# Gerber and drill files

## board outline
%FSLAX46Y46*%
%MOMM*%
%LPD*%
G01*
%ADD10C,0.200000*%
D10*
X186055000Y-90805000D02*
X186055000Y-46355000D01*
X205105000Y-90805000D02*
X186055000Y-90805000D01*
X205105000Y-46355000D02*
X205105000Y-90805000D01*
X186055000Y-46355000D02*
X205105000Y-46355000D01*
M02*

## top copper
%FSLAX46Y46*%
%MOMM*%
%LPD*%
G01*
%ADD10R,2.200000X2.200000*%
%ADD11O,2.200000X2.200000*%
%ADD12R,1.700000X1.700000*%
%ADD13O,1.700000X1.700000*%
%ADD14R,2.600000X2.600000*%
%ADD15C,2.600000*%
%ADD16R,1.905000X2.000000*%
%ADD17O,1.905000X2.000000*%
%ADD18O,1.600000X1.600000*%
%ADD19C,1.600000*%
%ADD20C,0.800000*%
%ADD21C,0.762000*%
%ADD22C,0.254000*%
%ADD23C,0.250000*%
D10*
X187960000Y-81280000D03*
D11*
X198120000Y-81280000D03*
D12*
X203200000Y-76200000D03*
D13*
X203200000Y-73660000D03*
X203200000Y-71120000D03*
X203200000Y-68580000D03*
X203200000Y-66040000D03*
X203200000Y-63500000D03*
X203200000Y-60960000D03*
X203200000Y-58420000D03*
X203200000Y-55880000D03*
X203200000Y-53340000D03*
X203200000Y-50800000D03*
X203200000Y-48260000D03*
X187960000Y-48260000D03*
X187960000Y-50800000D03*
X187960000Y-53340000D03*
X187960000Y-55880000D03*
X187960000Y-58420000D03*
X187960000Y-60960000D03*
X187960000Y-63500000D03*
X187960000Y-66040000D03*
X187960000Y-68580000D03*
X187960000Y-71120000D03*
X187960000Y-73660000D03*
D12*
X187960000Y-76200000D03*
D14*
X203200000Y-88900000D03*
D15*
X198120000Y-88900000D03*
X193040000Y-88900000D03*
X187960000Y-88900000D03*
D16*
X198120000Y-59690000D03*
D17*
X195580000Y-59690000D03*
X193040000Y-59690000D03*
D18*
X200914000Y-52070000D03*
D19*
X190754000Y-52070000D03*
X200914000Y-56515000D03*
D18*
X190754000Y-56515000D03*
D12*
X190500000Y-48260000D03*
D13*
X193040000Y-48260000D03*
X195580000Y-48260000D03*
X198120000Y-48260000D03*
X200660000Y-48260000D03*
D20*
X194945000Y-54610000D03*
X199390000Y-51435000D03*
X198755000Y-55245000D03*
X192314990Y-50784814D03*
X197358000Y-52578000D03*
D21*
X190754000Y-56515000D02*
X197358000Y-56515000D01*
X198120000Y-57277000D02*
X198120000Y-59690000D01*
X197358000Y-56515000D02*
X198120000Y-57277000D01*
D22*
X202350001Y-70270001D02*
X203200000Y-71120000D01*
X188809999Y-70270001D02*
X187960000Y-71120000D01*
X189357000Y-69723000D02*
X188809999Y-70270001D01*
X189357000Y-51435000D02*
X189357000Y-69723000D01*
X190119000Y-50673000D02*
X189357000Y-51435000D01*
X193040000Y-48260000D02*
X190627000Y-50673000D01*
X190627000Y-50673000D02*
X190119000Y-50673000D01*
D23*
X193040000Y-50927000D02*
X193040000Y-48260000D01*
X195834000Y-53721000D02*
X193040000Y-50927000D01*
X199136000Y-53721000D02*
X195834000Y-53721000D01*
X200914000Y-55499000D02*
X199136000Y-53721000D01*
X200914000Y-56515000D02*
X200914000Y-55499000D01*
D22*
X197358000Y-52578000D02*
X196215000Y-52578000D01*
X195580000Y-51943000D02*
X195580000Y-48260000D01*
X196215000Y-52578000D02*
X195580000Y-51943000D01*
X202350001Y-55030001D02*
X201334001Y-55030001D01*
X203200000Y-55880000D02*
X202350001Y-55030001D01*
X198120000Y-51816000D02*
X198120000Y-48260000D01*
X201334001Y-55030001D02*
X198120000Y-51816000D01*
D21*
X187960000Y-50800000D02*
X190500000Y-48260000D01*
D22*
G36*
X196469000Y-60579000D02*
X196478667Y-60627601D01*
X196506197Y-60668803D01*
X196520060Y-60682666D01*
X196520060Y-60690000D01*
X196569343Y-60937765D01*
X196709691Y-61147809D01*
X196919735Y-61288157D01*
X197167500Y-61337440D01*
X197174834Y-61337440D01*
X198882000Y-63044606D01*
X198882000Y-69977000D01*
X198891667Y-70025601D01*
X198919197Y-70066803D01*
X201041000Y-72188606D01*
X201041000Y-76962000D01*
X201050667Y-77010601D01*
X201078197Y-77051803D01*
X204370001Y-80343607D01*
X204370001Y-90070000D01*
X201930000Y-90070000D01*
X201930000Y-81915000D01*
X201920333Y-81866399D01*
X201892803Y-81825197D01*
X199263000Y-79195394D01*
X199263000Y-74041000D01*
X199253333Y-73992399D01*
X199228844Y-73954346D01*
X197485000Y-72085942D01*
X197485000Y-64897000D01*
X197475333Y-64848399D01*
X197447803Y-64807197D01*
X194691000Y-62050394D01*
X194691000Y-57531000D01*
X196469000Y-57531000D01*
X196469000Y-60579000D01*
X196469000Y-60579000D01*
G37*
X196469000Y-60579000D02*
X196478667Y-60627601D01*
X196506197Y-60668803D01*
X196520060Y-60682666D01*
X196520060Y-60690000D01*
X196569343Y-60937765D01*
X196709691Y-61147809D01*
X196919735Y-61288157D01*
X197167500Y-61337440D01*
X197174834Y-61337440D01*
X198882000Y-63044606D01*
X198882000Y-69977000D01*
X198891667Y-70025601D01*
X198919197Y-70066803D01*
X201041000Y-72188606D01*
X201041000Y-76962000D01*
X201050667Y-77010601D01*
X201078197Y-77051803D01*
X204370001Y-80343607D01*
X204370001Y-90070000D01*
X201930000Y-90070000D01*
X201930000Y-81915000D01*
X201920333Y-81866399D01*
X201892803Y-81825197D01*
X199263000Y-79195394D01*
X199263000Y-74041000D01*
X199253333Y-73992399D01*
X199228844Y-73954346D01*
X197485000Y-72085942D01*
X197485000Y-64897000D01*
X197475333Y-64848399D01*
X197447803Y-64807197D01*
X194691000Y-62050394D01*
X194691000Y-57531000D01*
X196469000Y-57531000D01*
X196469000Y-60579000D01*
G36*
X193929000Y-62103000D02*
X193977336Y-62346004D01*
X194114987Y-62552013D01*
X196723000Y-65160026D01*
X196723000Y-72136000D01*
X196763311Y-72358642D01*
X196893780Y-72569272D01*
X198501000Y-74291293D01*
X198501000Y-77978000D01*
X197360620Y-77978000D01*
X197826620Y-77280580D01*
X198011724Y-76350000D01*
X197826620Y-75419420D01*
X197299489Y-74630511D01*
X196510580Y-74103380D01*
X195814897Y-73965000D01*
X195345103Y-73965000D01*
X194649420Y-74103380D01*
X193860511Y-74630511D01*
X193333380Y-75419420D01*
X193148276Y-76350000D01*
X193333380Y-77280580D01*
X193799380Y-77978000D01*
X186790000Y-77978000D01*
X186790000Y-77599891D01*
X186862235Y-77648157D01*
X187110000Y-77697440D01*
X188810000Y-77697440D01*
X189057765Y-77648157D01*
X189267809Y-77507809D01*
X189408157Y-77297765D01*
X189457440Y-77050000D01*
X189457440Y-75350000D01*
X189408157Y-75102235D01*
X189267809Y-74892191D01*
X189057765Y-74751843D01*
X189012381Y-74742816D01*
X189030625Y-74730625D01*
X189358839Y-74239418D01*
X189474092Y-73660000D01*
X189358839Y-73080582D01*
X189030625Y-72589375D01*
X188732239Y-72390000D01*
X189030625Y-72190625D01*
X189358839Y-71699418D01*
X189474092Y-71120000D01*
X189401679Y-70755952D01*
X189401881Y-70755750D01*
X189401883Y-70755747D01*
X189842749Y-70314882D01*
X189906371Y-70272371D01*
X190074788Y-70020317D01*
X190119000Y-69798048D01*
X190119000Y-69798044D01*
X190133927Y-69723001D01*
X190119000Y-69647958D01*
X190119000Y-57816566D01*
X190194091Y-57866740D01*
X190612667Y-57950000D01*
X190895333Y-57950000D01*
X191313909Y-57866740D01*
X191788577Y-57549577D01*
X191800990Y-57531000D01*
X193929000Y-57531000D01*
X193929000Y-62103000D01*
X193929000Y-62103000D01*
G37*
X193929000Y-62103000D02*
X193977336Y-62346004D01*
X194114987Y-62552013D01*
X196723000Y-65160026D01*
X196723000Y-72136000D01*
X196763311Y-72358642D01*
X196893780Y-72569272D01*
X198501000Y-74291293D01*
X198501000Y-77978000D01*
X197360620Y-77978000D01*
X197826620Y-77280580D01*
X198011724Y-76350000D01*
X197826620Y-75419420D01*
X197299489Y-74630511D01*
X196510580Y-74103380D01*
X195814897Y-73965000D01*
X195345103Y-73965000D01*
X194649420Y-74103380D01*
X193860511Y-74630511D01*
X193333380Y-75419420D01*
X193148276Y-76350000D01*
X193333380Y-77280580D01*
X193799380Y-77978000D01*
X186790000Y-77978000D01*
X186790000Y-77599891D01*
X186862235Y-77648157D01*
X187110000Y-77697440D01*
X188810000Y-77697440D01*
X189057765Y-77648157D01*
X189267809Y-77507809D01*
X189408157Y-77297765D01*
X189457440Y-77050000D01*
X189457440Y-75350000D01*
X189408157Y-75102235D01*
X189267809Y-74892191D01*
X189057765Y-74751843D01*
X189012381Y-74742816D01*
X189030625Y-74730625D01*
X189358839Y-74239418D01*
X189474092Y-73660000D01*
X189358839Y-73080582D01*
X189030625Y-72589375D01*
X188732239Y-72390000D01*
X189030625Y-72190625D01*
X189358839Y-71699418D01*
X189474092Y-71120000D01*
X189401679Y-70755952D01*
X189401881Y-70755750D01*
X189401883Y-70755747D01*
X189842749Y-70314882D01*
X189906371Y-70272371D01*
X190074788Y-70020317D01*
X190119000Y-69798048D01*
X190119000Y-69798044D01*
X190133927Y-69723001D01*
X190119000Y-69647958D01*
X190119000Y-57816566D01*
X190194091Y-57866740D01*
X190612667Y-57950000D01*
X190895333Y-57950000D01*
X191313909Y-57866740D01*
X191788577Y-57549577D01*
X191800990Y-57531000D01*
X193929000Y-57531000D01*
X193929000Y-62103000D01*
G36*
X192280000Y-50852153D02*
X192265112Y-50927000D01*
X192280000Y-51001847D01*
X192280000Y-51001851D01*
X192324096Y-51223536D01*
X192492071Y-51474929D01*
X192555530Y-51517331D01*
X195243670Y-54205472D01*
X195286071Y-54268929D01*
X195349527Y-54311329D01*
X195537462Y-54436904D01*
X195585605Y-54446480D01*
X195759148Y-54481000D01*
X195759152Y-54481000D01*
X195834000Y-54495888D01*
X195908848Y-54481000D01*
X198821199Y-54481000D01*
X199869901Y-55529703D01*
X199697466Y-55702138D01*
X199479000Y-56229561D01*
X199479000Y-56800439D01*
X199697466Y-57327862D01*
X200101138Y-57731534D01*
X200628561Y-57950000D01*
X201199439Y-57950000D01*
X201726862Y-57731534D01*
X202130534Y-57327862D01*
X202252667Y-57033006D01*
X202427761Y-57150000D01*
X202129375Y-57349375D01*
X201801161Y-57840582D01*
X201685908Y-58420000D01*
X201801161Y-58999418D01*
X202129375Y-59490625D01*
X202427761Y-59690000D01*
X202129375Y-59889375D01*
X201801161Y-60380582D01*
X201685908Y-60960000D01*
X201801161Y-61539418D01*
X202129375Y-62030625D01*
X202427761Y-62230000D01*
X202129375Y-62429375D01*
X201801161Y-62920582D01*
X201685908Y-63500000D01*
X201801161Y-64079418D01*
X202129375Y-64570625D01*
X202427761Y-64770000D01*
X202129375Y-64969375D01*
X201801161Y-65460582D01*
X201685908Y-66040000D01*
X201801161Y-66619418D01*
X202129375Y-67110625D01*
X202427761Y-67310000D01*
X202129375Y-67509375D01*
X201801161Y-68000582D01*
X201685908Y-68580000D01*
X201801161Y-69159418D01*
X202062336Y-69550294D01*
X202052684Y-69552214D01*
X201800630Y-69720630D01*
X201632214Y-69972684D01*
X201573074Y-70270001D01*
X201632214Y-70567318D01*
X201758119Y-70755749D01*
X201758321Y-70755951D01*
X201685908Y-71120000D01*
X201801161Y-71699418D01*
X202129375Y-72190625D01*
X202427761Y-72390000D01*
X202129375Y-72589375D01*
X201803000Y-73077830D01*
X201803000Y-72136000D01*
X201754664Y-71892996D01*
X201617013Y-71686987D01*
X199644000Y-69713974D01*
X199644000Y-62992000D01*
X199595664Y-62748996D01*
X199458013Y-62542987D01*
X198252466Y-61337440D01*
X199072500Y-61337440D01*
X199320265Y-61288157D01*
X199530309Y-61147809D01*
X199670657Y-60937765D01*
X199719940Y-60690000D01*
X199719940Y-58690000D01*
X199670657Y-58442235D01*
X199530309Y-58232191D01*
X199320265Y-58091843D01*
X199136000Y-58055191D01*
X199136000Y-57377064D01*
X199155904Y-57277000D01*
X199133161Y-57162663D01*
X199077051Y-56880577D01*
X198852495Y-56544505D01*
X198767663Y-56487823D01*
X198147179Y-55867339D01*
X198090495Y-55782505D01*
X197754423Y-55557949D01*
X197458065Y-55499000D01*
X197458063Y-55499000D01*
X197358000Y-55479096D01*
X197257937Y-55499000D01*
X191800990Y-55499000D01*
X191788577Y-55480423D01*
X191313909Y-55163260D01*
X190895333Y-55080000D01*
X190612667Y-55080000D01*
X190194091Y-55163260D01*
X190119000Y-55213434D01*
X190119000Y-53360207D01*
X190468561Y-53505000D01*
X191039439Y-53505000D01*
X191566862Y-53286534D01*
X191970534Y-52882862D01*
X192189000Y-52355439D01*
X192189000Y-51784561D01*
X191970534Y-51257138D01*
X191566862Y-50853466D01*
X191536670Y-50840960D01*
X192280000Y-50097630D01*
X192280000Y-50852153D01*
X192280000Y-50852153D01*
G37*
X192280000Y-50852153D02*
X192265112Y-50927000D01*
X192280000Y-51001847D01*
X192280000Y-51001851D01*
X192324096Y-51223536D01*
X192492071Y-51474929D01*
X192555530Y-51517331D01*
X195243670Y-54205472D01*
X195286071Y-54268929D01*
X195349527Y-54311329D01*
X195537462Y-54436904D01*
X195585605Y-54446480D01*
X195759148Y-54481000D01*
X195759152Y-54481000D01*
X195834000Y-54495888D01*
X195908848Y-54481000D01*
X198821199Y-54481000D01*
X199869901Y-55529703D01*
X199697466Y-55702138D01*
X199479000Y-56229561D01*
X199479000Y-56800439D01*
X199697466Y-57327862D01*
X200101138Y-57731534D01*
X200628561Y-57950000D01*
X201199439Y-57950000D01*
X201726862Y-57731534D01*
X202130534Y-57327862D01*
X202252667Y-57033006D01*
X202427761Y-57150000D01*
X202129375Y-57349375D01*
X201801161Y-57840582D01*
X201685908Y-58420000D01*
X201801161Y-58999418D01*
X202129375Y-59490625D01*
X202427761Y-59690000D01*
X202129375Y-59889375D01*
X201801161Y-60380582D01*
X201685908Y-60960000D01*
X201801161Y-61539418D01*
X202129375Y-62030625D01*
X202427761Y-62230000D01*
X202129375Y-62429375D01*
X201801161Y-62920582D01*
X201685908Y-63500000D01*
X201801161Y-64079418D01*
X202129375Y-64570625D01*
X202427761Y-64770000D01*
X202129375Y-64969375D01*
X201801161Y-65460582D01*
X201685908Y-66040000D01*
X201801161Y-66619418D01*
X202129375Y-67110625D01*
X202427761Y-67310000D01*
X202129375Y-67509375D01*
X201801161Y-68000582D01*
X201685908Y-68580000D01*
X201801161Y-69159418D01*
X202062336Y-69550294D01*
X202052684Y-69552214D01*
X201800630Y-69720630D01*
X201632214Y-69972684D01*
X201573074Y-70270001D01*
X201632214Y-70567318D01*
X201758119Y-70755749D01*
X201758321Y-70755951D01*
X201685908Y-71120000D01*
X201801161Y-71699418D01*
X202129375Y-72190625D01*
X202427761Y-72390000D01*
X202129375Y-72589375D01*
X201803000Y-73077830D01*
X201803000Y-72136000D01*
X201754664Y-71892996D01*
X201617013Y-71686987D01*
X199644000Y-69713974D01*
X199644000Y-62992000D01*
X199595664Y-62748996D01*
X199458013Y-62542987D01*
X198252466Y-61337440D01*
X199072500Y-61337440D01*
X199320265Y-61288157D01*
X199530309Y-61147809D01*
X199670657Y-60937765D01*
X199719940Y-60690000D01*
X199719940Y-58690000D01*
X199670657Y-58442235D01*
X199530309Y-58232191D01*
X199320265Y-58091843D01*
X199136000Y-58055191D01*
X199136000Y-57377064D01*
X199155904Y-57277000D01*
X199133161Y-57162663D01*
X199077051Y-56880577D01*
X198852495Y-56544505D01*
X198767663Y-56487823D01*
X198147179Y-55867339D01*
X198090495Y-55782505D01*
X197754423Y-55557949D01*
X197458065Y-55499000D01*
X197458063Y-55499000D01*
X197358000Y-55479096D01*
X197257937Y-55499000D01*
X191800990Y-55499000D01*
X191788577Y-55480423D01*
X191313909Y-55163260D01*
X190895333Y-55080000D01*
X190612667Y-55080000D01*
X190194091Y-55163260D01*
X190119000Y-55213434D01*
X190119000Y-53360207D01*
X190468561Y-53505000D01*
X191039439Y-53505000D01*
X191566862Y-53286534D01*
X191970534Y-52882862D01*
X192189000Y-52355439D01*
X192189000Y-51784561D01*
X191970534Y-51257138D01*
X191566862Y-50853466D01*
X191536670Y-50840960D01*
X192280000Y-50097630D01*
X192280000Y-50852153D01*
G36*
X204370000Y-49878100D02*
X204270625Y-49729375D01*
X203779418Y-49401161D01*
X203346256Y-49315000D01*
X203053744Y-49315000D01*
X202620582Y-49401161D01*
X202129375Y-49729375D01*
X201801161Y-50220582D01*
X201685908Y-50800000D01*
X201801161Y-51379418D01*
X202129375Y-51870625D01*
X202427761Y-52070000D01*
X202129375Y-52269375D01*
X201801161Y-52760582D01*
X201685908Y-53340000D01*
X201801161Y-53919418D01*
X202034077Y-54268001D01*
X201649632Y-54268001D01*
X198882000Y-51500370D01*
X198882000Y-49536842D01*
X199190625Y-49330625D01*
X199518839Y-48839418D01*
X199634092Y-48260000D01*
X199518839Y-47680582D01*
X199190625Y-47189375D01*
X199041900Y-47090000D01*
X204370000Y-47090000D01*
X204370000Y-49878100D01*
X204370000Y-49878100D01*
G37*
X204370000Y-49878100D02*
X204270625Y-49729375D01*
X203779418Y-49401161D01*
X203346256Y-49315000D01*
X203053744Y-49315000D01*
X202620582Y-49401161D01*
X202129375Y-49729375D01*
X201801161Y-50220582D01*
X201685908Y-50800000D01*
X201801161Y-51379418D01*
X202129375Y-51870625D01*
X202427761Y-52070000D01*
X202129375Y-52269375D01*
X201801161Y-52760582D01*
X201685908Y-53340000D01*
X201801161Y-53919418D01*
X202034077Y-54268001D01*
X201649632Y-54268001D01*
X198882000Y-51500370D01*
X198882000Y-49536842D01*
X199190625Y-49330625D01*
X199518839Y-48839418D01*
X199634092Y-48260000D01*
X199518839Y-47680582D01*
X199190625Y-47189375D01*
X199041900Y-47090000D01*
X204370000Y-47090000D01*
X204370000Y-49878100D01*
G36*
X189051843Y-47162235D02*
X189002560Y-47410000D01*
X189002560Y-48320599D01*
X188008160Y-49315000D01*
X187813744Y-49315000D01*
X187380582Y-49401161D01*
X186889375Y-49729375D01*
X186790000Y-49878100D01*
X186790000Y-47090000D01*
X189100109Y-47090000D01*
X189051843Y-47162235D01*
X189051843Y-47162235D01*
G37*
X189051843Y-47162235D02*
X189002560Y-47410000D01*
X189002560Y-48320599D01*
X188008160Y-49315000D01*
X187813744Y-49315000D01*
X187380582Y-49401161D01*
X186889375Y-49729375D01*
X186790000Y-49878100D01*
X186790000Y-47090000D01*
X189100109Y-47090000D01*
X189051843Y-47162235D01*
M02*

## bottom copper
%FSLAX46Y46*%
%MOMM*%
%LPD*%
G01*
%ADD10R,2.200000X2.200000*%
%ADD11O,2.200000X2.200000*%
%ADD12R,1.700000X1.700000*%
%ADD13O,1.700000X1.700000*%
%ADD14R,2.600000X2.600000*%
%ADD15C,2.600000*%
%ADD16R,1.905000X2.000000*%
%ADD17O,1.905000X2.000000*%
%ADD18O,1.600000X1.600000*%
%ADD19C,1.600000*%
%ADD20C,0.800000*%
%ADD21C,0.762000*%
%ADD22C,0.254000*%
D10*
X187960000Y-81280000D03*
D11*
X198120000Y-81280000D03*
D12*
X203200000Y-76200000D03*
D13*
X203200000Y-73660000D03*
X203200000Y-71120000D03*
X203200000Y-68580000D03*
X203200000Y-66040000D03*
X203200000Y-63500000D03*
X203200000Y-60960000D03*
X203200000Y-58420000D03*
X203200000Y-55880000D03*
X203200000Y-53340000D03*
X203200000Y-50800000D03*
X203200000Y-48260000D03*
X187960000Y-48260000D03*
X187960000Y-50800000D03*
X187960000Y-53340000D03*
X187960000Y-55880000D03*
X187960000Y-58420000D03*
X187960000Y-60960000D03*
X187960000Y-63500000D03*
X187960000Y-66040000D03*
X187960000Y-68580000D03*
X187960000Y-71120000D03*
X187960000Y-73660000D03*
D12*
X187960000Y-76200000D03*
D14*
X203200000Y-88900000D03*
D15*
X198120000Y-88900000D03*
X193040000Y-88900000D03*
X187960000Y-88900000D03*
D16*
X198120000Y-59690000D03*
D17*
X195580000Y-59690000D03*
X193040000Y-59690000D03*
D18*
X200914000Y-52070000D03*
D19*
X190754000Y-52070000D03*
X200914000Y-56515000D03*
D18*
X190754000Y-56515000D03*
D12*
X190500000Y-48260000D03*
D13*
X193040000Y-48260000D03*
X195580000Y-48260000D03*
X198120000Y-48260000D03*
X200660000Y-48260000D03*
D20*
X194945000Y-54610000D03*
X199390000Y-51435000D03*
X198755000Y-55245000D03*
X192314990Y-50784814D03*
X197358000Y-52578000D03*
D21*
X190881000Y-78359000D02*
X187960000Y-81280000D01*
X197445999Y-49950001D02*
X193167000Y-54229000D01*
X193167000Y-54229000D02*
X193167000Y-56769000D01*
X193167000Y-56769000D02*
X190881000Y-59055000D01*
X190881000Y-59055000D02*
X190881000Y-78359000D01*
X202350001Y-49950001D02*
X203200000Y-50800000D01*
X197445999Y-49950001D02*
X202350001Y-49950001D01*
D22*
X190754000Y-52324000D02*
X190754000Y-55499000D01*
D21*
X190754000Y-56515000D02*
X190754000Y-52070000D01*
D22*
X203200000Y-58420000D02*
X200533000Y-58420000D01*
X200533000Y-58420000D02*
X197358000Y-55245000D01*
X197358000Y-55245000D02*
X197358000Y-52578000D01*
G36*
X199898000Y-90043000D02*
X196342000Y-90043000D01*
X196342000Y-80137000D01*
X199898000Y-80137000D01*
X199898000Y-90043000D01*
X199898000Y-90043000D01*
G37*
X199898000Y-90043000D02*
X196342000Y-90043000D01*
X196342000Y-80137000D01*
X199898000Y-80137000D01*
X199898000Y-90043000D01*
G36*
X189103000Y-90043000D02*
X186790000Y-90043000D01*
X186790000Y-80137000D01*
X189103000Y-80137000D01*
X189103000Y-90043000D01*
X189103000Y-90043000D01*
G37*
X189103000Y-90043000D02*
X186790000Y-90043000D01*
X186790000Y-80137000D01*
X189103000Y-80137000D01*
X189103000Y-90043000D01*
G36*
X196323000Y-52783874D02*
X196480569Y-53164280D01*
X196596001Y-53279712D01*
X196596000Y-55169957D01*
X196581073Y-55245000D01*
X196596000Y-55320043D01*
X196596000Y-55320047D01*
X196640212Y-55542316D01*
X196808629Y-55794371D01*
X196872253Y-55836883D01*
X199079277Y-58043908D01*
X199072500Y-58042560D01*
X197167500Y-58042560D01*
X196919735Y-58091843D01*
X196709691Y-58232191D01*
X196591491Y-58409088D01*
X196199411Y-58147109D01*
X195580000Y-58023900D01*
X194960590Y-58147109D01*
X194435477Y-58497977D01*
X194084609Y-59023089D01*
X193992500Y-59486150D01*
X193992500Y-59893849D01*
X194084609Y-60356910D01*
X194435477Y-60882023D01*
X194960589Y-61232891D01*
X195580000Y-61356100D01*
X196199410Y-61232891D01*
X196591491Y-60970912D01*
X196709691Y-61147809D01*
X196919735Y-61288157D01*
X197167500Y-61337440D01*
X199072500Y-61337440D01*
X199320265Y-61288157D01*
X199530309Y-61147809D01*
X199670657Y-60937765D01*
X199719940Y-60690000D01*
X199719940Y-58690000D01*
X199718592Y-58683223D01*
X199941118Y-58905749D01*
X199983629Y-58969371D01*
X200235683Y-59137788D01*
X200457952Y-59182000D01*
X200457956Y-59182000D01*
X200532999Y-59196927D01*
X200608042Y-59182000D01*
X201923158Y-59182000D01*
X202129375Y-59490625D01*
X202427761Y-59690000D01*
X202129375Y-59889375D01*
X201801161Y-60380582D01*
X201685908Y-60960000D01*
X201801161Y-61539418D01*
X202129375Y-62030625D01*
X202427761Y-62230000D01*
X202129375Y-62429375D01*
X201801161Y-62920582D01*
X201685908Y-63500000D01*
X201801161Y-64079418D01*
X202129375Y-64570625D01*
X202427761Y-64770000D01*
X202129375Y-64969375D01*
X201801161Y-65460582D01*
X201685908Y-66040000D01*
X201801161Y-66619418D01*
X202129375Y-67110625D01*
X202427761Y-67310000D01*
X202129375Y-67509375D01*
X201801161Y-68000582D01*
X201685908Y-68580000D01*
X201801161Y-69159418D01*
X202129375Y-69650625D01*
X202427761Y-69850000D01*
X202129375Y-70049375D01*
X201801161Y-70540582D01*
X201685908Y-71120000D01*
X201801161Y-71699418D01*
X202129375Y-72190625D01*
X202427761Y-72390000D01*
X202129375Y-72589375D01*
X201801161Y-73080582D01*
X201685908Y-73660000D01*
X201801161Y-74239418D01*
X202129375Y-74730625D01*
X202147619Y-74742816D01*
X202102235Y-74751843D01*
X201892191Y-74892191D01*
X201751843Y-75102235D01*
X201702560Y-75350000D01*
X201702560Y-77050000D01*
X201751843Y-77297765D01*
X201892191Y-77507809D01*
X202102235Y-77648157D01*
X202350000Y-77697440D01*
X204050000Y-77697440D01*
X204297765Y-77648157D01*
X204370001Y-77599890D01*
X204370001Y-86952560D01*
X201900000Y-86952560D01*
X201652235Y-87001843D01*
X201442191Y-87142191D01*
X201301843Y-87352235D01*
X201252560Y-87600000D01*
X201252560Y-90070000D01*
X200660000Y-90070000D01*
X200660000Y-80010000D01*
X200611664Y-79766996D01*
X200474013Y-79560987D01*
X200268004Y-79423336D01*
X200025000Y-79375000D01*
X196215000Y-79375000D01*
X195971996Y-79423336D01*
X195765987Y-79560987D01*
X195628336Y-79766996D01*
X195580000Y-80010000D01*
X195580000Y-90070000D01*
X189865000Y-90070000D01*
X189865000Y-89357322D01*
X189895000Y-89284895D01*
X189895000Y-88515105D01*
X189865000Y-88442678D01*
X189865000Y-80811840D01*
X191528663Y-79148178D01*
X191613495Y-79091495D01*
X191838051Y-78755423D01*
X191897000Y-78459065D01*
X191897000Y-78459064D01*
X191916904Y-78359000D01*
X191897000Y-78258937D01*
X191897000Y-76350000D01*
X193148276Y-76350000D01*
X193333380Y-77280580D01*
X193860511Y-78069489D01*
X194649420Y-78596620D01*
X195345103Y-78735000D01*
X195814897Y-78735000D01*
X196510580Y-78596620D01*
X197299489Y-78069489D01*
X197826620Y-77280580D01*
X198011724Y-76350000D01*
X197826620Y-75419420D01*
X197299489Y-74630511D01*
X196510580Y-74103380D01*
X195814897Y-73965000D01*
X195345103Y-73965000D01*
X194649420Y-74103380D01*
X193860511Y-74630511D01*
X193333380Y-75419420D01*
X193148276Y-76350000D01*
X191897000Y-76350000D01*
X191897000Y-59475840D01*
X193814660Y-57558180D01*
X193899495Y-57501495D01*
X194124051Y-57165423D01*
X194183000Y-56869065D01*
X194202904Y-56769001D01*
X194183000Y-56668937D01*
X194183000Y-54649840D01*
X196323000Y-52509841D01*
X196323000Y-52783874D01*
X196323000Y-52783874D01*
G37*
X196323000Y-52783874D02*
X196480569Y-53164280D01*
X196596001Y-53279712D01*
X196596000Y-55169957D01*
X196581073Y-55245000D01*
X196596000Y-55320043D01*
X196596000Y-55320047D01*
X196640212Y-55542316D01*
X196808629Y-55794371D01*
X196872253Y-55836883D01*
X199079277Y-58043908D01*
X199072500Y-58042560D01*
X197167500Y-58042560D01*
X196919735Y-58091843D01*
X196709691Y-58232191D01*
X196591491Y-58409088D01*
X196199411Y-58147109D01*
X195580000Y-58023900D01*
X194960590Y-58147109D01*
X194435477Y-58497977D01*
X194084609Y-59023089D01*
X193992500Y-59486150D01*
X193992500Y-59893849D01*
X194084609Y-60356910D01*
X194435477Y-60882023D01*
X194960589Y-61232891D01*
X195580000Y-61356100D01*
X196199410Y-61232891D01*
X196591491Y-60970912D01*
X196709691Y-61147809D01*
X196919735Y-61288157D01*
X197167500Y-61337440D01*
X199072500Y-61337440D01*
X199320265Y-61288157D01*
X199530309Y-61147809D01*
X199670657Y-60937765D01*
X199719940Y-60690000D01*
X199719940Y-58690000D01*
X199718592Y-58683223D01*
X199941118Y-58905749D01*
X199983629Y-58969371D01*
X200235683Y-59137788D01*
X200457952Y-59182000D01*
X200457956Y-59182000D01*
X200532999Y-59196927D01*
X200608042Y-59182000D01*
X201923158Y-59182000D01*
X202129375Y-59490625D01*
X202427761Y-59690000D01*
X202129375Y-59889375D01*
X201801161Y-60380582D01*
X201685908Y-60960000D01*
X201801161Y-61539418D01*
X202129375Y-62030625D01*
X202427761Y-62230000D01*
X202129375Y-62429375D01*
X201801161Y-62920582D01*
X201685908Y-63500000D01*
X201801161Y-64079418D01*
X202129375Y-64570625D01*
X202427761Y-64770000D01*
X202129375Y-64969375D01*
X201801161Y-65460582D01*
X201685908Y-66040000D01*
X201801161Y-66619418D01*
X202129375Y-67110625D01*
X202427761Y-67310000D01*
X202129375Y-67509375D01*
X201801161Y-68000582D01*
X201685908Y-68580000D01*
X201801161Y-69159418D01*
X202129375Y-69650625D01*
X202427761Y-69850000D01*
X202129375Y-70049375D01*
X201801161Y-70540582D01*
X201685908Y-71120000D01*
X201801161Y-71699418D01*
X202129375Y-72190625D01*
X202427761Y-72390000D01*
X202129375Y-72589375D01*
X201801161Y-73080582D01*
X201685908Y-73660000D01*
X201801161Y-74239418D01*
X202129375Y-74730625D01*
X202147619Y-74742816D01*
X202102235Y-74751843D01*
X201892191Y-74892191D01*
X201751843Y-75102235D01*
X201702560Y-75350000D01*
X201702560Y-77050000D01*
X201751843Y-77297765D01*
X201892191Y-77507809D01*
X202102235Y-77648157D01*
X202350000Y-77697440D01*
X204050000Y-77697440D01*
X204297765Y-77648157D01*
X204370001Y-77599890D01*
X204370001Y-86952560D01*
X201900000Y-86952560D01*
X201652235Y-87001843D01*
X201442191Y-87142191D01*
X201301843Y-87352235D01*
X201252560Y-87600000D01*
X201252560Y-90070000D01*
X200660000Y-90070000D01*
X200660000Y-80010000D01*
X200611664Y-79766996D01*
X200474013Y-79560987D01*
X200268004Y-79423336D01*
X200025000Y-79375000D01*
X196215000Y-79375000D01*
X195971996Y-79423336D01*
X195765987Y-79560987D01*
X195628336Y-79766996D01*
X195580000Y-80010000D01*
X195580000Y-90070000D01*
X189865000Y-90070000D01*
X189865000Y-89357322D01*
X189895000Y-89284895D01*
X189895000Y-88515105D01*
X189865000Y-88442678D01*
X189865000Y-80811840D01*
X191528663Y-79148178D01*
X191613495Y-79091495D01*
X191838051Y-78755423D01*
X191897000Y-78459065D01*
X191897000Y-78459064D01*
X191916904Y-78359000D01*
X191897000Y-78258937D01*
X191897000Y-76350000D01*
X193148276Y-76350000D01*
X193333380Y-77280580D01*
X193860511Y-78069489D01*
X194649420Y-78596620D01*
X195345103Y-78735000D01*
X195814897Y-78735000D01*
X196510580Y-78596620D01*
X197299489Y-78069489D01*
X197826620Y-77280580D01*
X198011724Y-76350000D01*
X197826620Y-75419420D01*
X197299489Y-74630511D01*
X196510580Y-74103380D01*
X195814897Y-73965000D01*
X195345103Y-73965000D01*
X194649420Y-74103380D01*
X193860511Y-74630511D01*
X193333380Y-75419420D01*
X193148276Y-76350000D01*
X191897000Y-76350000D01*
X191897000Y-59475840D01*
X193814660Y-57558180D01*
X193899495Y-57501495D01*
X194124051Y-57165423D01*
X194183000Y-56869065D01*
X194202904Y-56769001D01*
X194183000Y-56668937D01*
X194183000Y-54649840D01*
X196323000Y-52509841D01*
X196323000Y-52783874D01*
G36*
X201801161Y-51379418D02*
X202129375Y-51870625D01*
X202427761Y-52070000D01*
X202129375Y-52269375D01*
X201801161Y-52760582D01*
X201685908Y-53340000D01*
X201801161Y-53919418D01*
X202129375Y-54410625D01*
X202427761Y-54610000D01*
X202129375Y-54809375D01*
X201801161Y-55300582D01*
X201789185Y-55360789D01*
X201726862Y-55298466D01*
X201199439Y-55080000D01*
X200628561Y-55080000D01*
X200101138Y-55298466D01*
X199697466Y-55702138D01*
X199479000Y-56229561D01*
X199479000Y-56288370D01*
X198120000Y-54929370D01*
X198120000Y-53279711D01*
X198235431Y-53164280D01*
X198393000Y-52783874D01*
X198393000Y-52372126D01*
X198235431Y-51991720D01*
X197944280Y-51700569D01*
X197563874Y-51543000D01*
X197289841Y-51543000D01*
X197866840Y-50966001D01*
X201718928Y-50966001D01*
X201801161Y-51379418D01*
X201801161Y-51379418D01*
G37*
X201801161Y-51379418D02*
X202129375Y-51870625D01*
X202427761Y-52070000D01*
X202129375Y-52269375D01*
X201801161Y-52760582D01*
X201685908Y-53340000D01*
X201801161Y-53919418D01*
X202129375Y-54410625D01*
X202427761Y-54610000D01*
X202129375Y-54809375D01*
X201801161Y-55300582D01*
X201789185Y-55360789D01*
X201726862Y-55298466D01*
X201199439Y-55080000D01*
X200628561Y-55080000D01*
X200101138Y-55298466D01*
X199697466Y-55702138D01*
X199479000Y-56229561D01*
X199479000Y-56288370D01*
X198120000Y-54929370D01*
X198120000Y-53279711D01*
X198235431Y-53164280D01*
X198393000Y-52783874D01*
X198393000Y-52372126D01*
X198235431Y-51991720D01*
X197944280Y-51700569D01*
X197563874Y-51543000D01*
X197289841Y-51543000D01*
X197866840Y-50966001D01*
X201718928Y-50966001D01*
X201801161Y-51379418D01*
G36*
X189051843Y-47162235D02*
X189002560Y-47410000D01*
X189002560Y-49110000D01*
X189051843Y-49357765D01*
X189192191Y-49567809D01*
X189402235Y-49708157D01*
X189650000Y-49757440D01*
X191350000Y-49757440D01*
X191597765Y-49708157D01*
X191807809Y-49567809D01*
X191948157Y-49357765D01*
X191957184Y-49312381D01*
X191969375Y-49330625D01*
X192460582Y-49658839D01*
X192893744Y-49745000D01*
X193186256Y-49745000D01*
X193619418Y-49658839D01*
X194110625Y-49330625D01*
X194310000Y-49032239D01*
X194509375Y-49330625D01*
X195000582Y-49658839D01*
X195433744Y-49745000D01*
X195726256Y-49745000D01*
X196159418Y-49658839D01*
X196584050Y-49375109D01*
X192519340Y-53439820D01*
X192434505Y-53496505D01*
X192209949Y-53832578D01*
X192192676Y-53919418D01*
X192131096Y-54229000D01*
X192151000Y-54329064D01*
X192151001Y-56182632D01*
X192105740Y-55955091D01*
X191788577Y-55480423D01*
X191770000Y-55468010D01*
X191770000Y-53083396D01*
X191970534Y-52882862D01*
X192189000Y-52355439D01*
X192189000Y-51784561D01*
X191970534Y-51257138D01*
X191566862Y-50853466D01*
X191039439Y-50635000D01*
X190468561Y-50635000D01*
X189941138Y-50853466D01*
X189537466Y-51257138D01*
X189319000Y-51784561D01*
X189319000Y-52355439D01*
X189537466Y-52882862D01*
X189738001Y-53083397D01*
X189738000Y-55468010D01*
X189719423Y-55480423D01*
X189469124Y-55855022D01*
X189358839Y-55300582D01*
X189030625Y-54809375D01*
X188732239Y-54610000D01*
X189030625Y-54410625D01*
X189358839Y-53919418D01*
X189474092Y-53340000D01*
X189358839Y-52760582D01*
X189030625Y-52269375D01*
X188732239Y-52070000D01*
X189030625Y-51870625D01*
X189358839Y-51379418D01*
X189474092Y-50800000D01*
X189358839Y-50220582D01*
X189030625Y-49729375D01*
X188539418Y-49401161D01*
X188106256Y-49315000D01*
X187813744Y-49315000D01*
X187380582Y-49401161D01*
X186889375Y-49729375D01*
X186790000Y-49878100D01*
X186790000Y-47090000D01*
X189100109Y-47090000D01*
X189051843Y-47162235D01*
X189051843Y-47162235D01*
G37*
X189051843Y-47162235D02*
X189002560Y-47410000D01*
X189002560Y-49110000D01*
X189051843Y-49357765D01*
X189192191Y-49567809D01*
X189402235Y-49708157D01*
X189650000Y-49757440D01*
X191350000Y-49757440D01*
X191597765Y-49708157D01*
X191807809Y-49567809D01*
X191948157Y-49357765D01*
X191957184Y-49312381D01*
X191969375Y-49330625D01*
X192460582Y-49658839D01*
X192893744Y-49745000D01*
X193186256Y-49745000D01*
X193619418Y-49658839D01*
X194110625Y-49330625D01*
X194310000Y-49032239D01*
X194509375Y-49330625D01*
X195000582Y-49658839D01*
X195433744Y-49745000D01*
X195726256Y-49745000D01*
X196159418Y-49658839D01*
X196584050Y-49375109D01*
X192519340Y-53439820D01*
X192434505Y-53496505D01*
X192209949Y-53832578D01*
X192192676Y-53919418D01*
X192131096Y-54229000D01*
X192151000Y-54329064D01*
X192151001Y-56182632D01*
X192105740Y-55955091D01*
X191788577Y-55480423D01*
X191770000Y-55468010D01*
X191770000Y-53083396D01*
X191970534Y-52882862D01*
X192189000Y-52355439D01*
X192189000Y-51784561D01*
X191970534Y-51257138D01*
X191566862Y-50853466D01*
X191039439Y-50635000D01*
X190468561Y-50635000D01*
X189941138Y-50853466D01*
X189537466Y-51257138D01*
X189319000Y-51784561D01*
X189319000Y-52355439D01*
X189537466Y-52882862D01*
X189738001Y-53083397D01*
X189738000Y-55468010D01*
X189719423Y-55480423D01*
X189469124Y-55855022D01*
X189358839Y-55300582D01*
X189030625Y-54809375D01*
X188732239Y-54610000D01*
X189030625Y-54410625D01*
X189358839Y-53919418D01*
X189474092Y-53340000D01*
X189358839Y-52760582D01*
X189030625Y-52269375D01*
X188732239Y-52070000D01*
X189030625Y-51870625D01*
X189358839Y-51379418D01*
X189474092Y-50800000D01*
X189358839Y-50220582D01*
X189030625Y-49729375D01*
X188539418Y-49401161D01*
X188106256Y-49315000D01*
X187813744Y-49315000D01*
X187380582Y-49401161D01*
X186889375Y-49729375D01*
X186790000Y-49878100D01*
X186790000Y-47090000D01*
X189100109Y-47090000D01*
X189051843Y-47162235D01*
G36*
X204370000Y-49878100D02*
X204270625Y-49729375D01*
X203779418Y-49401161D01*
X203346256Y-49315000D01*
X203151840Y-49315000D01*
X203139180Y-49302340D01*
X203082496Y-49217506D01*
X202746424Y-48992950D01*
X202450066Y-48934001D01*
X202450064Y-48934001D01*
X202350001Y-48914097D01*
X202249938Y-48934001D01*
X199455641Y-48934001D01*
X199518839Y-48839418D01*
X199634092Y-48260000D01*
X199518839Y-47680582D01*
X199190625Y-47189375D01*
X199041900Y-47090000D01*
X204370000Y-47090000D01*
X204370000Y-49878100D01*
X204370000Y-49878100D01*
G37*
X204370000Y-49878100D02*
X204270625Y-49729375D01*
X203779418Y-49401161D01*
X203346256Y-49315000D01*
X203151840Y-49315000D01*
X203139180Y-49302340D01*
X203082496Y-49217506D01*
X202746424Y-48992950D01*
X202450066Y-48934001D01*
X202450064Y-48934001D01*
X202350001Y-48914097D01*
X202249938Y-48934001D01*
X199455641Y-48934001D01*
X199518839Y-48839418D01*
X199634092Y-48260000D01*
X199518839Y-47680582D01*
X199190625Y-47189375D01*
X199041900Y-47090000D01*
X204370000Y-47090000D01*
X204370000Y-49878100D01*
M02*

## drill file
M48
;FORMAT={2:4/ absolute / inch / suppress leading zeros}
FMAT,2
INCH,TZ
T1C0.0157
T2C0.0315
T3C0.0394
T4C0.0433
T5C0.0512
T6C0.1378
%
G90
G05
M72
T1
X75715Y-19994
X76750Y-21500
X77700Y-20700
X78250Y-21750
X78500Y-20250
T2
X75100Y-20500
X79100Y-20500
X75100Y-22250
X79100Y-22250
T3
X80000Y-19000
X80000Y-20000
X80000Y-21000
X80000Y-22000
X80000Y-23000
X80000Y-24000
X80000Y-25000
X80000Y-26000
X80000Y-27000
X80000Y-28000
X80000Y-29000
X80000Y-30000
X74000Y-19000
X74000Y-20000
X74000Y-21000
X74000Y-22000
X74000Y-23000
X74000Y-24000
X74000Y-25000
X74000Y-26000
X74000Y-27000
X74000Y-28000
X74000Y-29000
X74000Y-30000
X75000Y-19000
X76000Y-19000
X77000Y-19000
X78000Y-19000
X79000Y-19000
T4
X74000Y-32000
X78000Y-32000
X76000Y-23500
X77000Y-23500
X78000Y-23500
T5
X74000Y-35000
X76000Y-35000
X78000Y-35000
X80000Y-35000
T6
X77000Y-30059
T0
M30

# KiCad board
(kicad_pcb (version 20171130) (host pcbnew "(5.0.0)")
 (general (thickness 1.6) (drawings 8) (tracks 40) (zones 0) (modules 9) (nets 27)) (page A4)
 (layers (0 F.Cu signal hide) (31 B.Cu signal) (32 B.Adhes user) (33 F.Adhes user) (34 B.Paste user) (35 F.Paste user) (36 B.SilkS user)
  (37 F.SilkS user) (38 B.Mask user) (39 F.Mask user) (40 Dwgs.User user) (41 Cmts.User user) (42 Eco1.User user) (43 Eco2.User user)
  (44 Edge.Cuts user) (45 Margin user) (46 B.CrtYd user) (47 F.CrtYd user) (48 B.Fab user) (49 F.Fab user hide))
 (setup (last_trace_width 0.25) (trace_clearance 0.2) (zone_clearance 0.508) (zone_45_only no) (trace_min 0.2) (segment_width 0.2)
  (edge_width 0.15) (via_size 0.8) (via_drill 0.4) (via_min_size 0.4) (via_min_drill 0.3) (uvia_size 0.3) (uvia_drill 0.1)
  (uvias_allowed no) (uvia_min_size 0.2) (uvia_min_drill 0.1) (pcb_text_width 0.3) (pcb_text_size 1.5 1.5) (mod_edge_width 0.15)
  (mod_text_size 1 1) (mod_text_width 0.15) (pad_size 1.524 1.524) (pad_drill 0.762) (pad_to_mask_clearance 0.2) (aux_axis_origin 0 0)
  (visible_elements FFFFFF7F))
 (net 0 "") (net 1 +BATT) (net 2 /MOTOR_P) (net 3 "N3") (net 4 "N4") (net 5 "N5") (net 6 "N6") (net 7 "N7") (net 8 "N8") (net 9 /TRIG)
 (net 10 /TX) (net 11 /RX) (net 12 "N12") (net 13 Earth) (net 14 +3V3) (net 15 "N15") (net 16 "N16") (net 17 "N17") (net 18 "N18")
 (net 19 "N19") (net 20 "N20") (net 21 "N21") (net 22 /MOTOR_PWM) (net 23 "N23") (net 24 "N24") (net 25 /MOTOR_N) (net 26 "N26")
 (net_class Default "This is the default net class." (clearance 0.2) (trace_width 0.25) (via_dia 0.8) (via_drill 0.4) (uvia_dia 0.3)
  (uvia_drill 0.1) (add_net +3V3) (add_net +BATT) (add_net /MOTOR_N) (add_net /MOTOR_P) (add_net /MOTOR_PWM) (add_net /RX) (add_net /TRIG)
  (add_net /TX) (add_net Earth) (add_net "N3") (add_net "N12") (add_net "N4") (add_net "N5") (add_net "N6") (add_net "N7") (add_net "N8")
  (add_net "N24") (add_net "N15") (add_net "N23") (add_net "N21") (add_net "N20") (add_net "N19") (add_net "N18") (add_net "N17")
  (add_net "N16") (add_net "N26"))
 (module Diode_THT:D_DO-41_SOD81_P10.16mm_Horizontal (layer F.Cu) (at 187.96 81.28)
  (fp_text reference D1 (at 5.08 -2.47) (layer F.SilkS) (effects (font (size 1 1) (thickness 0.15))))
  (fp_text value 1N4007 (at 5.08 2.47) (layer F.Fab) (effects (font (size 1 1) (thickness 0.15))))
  (pad 1 thru_hole rect (at 0 0) (size 2.2 2.2) (drill 1.1) (layers *.Cu *.Mask) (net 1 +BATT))
  (pad 2 thru_hole oval (at 10.16 0) (size 2.2 2.2) (drill 1.1) (layers *.Cu *.Mask) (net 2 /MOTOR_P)))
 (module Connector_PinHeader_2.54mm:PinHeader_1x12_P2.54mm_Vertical (layer F.Cu) (at 203.2 76.2 180)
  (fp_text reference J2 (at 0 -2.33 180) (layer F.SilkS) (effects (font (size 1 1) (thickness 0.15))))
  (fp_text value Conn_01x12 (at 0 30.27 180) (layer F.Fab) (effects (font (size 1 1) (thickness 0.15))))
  (pad 1 thru_hole rect (at 0 0 180) (size 1.7 1.7) (drill 1) (layers *.Cu *.Mask) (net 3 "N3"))
  (pad 2 thru_hole oval (at 0 2.54 180) (size 1.7 1.7) (drill 1) (layers *.Cu *.Mask) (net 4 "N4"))
  (pad 3 thru_hole oval (at 0 5.08 180) (size 1.7 1.7) (drill 1) (layers *.Cu *.Mask) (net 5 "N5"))
  (pad 4 thru_hole oval (at 0 7.62 180) (size 1.7 1.7) (drill 1) (layers *.Cu *.Mask) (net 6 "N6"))
  (pad 5 thru_hole oval (at 0 10.16 180) (size 1.7 1.7) (drill 1) (layers *.Cu *.Mask) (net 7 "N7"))
  (pad 6 thru_hole oval (at 0 12.7 180) (size 1.7 1.7) (drill 1) (layers *.Cu *.Mask) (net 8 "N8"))
  (pad 7 thru_hole oval (at 0 15.24 180) (size 1.7 1.7) (drill 1) (layers *.Cu *.Mask) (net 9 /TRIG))
  (pad 8 thru_hole oval (at 0 17.78 180) (size 1.7 1.7) (drill 1) (layers *.Cu *.Mask) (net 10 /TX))
  (pad 9 thru_hole oval (at 0 20.32 180) (size 1.7 1.7) (drill 1) (layers *.Cu *.Mask) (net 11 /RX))
  (pad 10 thru_hole oval (at 0 22.86 180) (size 1.7 1.7) (drill 1) (layers *.Cu *.Mask) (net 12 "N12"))
  (pad 11 thru_hole oval (at 0 25.4 180) (size 1.7 1.7) (drill 1) (layers *.Cu *.Mask) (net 1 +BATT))
  (pad 12 thru_hole oval (at 0 27.94 180) (size 1.7 1.7) (drill 1) (layers *.Cu *.Mask) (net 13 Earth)))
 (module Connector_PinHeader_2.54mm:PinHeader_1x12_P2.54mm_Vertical (layer F.Cu) (at 187.96 76.2 180)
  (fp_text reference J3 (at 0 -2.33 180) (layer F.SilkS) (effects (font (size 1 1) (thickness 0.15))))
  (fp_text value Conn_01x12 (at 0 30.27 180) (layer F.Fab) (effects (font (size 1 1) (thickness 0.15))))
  (pad 12 thru_hole oval (at 0 27.94 180) (size 1.7 1.7) (drill 1) (layers *.Cu *.Mask) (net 13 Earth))
  (pad 11 thru_hole oval (at 0 25.4 180) (size 1.7 1.7) (drill 1) (layers *.Cu *.Mask) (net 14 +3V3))
  (pad 10 thru_hole oval (at 0 22.86 180) (size 1.7 1.7) (drill 1) (layers *.Cu *.Mask) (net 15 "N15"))
  (pad 9 thru_hole oval (at 0 20.32 180) (size 1.7 1.7) (drill 1) (layers *.Cu *.Mask) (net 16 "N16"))
  (pad 8 thru_hole oval (at 0 17.78 180) (size 1.7 1.7) (drill 1) (layers *.Cu *.Mask) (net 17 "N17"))
  (pad 7 thru_hole oval (at 0 15.24 180) (size 1.7 1.7) (drill 1) (layers *.Cu *.Mask) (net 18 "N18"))
  (pad 6 thru_hole oval (at 0 12.7 180) (size 1.7 1.7) (drill 1) (layers *.Cu *.Mask) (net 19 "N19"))
  (pad 5 thru_hole oval (at 0 10.16 180) (size 1.7 1.7) (drill 1) (layers *.Cu *.Mask) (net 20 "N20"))
  (pad 4 thru_hole oval (at 0 7.62 180) (size 1.7 1.7) (drill 1) (layers *.Cu *.Mask) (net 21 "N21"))
  (pad 3 thru_hole oval (at 0 5.08 180) (size 1.7 1.7) (drill 1) (layers *.Cu *.Mask) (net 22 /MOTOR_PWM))
  (pad 2 thru_hole oval (at 0 2.54 180) (size 1.7 1.7) (drill 1) (layers *.Cu *.Mask) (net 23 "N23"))
  (pad 1 thru_hole rect (at 0 0 180) (size 1.7 1.7) (drill 1) (layers *.Cu *.Mask) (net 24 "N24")))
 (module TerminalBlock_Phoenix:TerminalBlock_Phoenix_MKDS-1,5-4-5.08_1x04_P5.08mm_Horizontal (layer F.Cu) (at 203.2 88.9 180)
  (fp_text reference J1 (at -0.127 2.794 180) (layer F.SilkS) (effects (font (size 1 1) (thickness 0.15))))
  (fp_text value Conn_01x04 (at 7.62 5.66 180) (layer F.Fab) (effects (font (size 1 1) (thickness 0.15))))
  (pad 1 thru_hole rect (at 0 0 180) (size 2.6 2.6) (drill 1.3) (layers *.Cu *.Mask) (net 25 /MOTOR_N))
  (pad 2 thru_hole circle (at 5.08 0 180) (size 2.6 2.6) (drill 1.3) (layers *.Cu *.Mask) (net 2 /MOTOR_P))
  (pad 3 thru_hole circle (at 10.16 0 180) (size 2.6 2.6) (drill 1.3) (layers *.Cu *.Mask) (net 13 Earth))
  (pad 4 thru_hole circle (at 15.24 0 180) (size 2.6 2.6) (drill 1.3) (layers *.Cu *.Mask) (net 1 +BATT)))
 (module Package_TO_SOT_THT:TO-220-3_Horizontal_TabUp (layer B.Cu) (at 198.12 59.69 180)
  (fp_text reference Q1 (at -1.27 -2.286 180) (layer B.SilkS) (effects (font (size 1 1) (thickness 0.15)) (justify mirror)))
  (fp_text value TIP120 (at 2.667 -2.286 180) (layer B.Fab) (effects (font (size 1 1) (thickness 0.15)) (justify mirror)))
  (pad "" np_thru_hole oval (at 2.54 -16.66 180) (size 3.5 3.5) (drill 3.5) (layers *.Cu *.Mask))
  (pad 1 thru_hole rect (at 0 0 180) (size 1.905 2) (drill 1.1) (layers *.Cu *.Mask) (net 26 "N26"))
  (pad 2 thru_hole oval (at 2.54 0 180) (size 1.905 2) (drill 1.1) (layers *.Cu *.Mask) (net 25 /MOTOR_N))
  (pad 3 thru_hole oval (at 5.08 0 180) (size 1.905 2) (drill 1.1) (layers *.Cu *.Mask) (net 13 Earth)))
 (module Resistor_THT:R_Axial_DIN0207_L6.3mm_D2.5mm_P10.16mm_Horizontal (layer F.Cu) (at 190.754 52.07)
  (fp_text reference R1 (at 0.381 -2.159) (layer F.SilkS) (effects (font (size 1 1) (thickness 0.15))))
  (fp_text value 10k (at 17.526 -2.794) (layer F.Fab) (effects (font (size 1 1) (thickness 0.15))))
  (pad 2 thru_hole oval (at 10.16 0) (size 1.6 1.6) (drill 0.8) (layers *.Cu *.Mask) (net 13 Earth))
  (pad 1 thru_hole circle (at 0 0) (size 1.6 1.6) (drill 0.8) (layers *.Cu *.Mask) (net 26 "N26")))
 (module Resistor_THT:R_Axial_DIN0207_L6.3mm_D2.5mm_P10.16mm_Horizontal (layer F.Cu) (at 200.914 56.515 180)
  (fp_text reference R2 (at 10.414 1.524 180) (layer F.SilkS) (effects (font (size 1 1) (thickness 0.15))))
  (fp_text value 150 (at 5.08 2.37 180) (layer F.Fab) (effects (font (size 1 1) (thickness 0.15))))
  (pad 1 thru_hole circle (at 0 0 180) (size 1.6 1.6) (drill 0.8) (layers *.Cu *.Mask) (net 22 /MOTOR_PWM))
  (pad 2 thru_hole oval (at 10.16 0 180) (size 1.6 1.6) (drill 0.8) (layers *.Cu *.Mask) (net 26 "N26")))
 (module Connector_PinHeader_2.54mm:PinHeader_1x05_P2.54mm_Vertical (layer F.Cu) (at 190.5 48.26 90)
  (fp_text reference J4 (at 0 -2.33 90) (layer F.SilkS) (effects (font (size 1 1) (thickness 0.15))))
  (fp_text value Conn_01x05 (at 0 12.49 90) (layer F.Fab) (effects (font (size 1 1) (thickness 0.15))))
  (pad 1 thru_hole rect (at 0 0 90) (size 1.7 1.7) (drill 1) (layers *.Cu *.Mask) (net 14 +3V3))
  (pad 2 thru_hole oval (at 0 2.54 90) (size 1.7 1.7) (drill 1) (layers *.Cu *.Mask) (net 22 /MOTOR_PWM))
  (pad 3 thru_hole oval (at 0 5.08 90) (size 1.7 1.7) (drill 1) (layers *.Cu *.Mask) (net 10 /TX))
  (pad 4 thru_hole oval (at 0 7.62 90) (size 1.7 1.7) (drill 1) (layers *.Cu *.Mask) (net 11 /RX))
  (pad 5 thru_hole oval (at 0 10.16 90) (size 1.7 1.7) (drill 1) (layers *.Cu *.Mask) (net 13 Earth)))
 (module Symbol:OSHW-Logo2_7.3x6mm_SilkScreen (layer B.Cu) (at 195.707 67.564 180)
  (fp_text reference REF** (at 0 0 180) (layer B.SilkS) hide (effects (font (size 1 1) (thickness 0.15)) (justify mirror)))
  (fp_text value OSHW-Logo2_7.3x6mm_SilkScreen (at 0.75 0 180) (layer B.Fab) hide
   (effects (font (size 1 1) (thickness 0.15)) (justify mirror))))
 (gr_line (start 186.055 90.805) (end 186.055 46.355) (layer Edge.Cuts) (width 0.2))
 (gr_line (start 205.105 90.805) (end 186.055 90.805) (layer Edge.Cuts) (width 0.2))
 (gr_line (start 205.105 46.355) (end 205.105 90.805) (layer Edge.Cuts) (width 0.2))
 (gr_line (start 186.055 46.355) (end 205.105 46.355) (layer Edge.Cuts) (width 0.2))
 (segment (start 190.881 78.359) (end 187.96 81.28) (width 0.762) (layer B.Cu) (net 1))
 (segment (start 197.445999 49.950001) (end 193.167 54.229) (width 0.762) (layer B.Cu) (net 1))
 (segment (start 193.167 54.229) (end 193.167 56.769) (width 0.762) (layer B.Cu) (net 1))
 (segment (start 193.167 56.769) (end 190.881 59.055) (width 0.762) (layer B.Cu) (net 1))
 (segment (start 190.881 59.055) (end 190.881 78.359) (width 0.762) (layer B.Cu) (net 1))
 (segment (start 202.350001 49.950001) (end 203.2 50.8) (width 0.762) (layer B.Cu) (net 1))
 (segment (start 197.445999 49.950001) (end 202.350001 49.950001) (width 0.762) (layer B.Cu) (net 1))
 (segment (start 190.754 52.324) (end 190.754 55.499) (width 0.254) (layer B.Cu) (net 26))
 (segment (start 190.754 56.515) (end 197.358 56.515) (width 0.762) (layer F.Cu) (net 26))
 (segment (start 198.12 57.277) (end 198.12 59.69) (width 0.762) (layer F.Cu) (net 26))
 (segment (start 197.358 56.515) (end 198.12 57.277) (width 0.762) (layer F.Cu) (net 26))
 (segment (start 190.754 56.515) (end 190.754 52.07) (width 0.762) (layer B.Cu) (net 26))
 (via (at 194.945 54.61) (size 0.8) (drill 0.4) (layers F.Cu B.Cu) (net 13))
 (via (at 199.39 51.435) (size 0.8) (drill 0.4) (layers F.Cu B.Cu) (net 13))
 (via (at 198.755 55.245) (size 0.8) (drill 0.4) (layers F.Cu B.Cu) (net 13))
 (via (at 192.31499 50.784814) (size 0.8) (drill 0.4) (layers F.Cu B.Cu) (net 13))
 (segment (start 202.350001 70.270001) (end 203.2 71.12) (width 0.254) (layer F.Cu) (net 5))
 (segment (start 188.809999 70.270001) (end 187.96 71.12) (width 0.254) (layer F.Cu) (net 22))
 (segment (start 189.357 69.723) (end 188.809999 70.270001) (width 0.254) (layer F.Cu) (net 22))
 (segment (start 189.357 51.435) (end 189.357 69.723) (width 0.254) (layer F.Cu) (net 22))
 (segment (start 190.119 50.673) (end 189.357 51.435) (width 0.254) (layer F.Cu) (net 22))
 (segment (start 193.04 48.26) (end 190.627 50.673) (width 0.254) (layer F.Cu) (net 22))
 (segment (start 190.627 50.673) (end 190.119 50.673) (width 0.254) (layer F.Cu) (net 22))
 (segment (start 193.04 50.927) (end 193.04 48.26) (width 0.25) (layer F.Cu) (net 22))
 (segment (start 195.834 53.721) (end 193.04 50.927) (width 0.25) (layer F.Cu) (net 22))
 (segment (start 199.136 53.721) (end 195.834 53.721) (width 0.25) (layer F.Cu) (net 22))
 (segment (start 200.914 55.499) (end 199.136 53.721) (width 0.25) (layer F.Cu) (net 22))
 (segment (start 200.914 56.515) (end 200.914 55.499) (width 0.25) (layer F.Cu) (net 22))
 (segment (start 203.2 58.42) (end 200.533 58.42) (width 0.254) (layer B.Cu) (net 10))
 (segment (start 200.533 58.42) (end 197.358 55.245) (width 0.254) (layer B.Cu) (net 10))
 (via (at 197.358 52.578) (size 0.8) (drill 0.4) (layers F.Cu B.Cu) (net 10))
 (segment (start 197.358 55.245) (end 197.358 52.578) (width 0.254) (layer B.Cu) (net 10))
 (segment (start 197.358 52.578) (end 196.215 52.578) (width 0.254) (layer F.Cu) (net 10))
 (segment (start 195.58 51.943) (end 195.58 48.26) (width 0.254) (layer F.Cu) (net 10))
 (segment (start 196.215 52.578) (end 195.58 51.943) (width 0.254) (layer F.Cu) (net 10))
 (segment (start 202.350001 55.030001) (end 201.334001 55.030001) (width 0.254) (layer F.Cu) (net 11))
 (segment (start 203.2 55.88) (end 202.350001 55.030001) (width 0.254) (layer F.Cu) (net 11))
 (segment (start 198.12 51.816) (end 198.12 48.26) (width 0.254) (layer F.Cu) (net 11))
 (segment (start 201.334001 55.030001) (end 198.12 51.816) (width 0.254) (layer F.Cu) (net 11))
 (segment (start 187.96 50.8) (end 190.5 48.26) (width 0.762) (layer F.Cu) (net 14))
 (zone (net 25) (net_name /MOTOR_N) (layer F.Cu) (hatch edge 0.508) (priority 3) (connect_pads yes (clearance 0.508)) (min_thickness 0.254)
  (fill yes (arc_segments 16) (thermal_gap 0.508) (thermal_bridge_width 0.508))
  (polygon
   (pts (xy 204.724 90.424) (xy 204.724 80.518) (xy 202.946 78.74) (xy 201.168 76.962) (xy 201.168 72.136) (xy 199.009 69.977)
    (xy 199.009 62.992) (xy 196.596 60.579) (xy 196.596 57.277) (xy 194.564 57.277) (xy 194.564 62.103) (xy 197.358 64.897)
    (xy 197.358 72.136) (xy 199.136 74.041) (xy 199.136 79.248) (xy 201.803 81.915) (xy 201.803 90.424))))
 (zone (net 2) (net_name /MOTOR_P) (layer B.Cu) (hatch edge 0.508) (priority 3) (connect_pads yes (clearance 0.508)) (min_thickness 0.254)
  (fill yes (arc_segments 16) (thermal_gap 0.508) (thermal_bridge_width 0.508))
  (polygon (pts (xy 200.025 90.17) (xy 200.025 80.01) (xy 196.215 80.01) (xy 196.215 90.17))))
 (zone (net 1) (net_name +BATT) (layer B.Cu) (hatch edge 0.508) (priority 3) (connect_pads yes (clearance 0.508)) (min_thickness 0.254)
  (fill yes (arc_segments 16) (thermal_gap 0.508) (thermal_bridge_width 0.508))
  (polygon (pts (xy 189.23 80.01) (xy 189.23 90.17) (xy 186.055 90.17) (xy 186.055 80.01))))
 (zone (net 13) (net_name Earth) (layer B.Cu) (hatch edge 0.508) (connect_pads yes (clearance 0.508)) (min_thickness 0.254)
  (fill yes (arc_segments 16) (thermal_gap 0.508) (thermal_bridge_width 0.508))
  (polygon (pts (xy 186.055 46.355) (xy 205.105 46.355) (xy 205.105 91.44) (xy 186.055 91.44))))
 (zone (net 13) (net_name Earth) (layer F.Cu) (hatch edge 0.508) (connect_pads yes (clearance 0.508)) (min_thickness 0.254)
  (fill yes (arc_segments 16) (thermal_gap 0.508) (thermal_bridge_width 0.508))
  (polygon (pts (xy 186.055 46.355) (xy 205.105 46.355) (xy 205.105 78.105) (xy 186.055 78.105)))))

